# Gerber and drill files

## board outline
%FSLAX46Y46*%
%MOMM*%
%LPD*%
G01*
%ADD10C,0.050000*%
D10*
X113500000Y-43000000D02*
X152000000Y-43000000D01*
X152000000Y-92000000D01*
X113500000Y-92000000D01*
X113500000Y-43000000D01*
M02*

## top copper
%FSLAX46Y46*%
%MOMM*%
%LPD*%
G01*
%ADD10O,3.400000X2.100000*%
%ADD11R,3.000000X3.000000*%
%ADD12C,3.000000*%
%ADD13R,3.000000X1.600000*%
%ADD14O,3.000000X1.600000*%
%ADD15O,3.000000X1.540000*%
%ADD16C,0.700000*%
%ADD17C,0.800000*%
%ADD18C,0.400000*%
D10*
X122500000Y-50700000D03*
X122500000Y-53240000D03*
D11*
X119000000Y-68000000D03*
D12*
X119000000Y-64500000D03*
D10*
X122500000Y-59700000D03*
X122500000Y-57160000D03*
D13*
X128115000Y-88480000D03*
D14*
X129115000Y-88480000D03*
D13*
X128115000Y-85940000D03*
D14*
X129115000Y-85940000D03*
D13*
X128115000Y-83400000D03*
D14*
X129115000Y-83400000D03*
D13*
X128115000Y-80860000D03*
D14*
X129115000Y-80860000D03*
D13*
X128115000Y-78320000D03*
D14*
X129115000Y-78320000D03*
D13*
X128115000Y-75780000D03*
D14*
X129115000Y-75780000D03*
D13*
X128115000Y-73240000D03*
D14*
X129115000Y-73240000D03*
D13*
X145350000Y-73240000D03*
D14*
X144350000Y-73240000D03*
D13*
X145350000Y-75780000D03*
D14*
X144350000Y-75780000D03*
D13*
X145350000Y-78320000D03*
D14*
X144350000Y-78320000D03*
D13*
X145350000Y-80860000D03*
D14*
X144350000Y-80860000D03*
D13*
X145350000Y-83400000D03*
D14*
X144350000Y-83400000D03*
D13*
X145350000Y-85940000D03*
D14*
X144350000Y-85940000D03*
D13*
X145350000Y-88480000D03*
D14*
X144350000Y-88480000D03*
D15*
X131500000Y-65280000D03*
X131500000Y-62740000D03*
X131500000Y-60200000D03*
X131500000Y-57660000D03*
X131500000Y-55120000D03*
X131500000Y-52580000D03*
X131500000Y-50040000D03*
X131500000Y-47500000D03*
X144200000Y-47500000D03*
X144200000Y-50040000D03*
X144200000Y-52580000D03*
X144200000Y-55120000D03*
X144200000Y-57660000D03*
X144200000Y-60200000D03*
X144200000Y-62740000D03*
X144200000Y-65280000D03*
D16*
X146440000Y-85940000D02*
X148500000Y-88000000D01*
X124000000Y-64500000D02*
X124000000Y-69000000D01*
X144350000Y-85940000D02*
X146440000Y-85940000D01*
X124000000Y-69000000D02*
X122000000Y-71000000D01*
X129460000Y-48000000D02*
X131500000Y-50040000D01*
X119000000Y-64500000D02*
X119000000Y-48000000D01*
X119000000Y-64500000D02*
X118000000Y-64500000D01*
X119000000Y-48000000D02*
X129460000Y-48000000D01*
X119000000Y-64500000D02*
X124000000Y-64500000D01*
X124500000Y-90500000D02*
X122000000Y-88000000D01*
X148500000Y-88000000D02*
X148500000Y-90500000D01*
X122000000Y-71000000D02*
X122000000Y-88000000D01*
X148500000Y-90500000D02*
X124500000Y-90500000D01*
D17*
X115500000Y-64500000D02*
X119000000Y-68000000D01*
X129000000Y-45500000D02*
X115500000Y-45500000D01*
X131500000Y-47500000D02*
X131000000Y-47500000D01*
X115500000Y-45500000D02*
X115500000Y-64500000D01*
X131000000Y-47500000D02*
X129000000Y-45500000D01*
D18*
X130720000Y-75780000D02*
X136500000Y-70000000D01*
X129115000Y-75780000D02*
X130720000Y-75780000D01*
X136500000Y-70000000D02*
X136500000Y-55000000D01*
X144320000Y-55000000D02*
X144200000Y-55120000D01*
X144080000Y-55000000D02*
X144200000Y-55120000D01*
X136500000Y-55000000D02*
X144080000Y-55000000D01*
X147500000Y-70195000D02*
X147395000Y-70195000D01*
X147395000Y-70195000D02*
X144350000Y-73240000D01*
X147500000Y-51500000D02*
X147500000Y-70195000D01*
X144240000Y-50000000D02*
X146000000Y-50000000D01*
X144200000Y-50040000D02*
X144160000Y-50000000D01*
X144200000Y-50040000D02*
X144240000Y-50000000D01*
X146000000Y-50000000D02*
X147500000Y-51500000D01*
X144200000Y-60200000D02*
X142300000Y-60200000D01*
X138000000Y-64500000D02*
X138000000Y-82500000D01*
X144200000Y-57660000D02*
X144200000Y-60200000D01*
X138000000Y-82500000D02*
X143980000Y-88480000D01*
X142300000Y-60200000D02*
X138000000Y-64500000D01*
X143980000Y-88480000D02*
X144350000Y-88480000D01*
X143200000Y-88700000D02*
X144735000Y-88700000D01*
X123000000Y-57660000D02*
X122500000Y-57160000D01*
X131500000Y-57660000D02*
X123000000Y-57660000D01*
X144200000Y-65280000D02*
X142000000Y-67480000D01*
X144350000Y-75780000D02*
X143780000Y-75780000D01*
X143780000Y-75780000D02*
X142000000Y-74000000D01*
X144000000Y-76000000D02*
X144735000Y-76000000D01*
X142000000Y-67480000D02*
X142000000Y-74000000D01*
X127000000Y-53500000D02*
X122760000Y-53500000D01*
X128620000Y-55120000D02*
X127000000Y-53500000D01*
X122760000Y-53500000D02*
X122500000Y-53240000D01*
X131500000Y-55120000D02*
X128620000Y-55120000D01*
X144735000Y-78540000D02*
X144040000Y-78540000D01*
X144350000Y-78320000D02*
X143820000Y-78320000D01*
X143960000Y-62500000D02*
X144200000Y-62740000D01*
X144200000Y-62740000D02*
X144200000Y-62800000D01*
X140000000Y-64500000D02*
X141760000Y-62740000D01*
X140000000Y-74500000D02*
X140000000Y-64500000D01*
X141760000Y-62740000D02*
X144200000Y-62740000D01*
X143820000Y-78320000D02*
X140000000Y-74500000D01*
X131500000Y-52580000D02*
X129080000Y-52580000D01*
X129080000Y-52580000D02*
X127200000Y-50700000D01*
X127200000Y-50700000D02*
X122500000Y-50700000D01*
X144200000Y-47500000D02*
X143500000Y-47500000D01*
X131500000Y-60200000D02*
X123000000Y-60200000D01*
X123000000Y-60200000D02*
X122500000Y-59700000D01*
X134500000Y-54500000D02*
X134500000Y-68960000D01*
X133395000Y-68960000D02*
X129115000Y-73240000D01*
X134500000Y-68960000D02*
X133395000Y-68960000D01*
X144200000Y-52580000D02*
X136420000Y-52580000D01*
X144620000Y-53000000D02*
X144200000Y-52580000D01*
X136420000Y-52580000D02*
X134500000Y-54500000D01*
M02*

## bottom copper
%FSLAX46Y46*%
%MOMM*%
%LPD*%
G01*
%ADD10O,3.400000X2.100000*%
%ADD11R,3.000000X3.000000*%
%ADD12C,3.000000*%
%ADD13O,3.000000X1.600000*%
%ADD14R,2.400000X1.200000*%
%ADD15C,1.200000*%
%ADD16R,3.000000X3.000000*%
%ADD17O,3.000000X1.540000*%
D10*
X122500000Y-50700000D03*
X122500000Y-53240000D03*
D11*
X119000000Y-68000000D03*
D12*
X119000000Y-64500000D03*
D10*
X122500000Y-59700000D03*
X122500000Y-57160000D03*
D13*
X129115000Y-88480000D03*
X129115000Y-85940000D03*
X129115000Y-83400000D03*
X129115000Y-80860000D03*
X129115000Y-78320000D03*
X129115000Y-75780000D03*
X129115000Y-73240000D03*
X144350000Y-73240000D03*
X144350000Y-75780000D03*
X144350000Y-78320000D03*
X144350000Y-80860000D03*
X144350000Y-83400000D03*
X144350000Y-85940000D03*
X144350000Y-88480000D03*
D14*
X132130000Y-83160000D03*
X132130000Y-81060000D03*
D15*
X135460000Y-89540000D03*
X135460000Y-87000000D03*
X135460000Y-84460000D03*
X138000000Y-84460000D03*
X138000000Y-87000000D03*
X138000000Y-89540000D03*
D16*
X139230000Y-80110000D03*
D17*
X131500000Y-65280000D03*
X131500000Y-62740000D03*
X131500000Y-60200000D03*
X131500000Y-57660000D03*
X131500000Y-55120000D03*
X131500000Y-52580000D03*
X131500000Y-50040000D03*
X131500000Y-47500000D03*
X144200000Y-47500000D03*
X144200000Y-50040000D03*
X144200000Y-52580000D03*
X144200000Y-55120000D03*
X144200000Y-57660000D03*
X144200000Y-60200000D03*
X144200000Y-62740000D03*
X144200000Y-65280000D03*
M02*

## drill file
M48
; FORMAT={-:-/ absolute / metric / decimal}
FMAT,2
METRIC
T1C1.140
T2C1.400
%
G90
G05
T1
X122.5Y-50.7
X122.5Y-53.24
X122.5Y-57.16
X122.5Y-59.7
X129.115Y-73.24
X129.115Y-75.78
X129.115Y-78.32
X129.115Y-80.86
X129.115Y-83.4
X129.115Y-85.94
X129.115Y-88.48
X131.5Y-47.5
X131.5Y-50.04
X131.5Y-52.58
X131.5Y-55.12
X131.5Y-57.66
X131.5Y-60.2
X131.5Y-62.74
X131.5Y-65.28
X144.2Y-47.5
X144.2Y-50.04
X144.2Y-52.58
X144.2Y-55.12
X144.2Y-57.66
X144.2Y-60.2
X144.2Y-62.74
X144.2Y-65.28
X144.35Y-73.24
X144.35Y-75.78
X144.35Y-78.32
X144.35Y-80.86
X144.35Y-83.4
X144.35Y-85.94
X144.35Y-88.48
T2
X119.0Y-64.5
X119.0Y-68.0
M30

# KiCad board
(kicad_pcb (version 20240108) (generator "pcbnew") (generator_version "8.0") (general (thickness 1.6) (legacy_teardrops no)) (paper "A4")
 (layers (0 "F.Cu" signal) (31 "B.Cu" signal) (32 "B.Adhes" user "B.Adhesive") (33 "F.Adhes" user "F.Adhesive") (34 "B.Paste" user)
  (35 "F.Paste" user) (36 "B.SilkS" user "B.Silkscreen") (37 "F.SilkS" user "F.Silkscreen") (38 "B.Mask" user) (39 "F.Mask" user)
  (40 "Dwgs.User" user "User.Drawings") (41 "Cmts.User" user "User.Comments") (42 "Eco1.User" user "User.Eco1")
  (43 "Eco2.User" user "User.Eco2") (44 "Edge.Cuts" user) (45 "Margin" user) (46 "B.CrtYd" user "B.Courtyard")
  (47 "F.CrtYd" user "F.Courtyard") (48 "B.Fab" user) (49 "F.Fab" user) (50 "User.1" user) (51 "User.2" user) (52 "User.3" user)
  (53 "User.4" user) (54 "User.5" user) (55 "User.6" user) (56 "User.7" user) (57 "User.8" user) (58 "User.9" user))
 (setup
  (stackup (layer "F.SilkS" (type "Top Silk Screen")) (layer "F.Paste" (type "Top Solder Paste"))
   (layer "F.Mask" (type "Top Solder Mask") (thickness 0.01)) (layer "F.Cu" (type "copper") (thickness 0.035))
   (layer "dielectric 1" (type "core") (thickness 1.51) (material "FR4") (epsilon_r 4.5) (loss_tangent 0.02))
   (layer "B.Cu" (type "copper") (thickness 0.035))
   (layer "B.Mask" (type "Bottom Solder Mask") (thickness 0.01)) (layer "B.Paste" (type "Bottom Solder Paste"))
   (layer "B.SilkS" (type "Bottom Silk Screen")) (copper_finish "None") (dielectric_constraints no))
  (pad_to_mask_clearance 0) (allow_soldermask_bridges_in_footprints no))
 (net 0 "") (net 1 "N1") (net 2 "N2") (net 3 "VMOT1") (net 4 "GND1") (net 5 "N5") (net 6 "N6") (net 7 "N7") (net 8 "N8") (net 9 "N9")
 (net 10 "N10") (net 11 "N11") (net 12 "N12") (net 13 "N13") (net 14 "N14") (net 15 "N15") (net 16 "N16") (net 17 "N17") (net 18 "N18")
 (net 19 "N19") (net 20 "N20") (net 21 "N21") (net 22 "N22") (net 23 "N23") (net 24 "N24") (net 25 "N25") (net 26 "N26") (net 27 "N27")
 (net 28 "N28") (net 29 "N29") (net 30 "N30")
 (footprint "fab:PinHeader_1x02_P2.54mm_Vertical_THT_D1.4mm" (layer "F.Cu") (at 122.5 50.7)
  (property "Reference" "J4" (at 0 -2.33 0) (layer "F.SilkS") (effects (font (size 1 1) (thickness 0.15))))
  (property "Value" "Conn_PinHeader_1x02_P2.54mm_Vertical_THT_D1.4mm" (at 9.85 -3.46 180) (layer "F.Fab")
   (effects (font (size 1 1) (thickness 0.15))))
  (pad "1" thru_hole oval (at 0 0) (size 3.4 2.1) (drill 1.14) (layers "*.Cu" "*.Mask") (remove_unused_layers no) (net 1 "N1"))
  (pad "2" thru_hole oval (at 0 2.54) (size 3.4 2.1) (drill 1.14) (layers "*.Cu" "*.Mask") (remove_unused_layers no) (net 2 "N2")))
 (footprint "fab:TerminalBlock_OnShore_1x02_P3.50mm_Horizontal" (layer "F.Cu") (at 119 68 90)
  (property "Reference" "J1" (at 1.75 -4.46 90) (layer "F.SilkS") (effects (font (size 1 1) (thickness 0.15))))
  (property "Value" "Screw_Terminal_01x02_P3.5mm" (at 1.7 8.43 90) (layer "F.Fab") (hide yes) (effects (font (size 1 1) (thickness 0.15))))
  (pad "1" thru_hole rect (at 0 0 90) (size 3 3) (drill 1.4) (layers "*.Cu" "*.Mask") (remove_unused_layers no) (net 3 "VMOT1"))
  (pad "2" thru_hole circle (at 3.5 0 90) (size 3 3) (drill 1.4) (layers "*.Cu" "*.Mask") (remove_unused_layers no) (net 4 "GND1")))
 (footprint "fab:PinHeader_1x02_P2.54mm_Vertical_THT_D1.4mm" (layer "F.Cu") (at 122.5 59.7 180)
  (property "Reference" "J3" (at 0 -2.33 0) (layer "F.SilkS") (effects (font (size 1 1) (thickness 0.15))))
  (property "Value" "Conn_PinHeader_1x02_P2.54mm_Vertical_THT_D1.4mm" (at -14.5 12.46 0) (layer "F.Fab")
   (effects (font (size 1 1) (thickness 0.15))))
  (pad "1" thru_hole oval (at 0 0 180) (size 3.4 2.1) (drill 1.14) (layers "*.Cu" "*.Mask") (remove_unused_layers no) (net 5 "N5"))
  (pad "2" thru_hole oval (at 0 2.54 180) (size 3.4 2.1) (drill 1.14) (layers "*.Cu" "*.Mask") (remove_unused_layers no) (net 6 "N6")))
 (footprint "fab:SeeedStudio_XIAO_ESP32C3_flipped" (layer "B.Cu") (at 136.73 80.86)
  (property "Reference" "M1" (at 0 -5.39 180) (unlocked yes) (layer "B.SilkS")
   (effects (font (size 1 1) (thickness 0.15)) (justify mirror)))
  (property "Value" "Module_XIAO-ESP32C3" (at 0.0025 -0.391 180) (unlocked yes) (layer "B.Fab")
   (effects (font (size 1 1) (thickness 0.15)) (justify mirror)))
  (pad "1" smd rect (at -7.615 7.62) (size 3 1.6) (drill (offset -1 0)) (layers "F.Cu" "F.Paste" "F.Mask") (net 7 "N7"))
  (pad "1" thru_hole oval (at -7.615 7.62) (size 3 1.6) (drill 1.14) (layers "*.Cu" "*.Mask") (remove_unused_layers no) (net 7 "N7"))
  (pad "2" smd rect (at -7.615 5.08) (size 3 1.6) (drill (offset -1 0)) (layers "F.Cu" "F.Paste" "F.Mask") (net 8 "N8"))
  (pad "2" thru_hole oval (at -7.615 5.08) (size 3 1.6) (drill 1.14) (layers "*.Cu" "*.Mask") (remove_unused_layers no) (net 8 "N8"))
  (pad "3" smd rect (at -7.615 2.54) (size 3 1.6) (drill (offset -1 0)) (layers "F.Cu" "F.Paste" "F.Mask") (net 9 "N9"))
  (pad "3" thru_hole oval (at -7.615 2.54) (size 3 1.6) (drill 1.14) (layers "*.Cu" "*.Mask") (remove_unused_layers no) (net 9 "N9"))
  (pad "4" smd rect (at -7.615 0) (size 3 1.6) (drill (offset -1 0)) (layers "F.Cu" "F.Paste" "F.Mask") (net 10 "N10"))
  (pad "4" thru_hole oval (at -7.615 0) (size 3 1.6) (drill 1.14) (layers "*.Cu" "*.Mask") (remove_unused_layers no) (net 10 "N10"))
  (pad "5" smd rect (at -7.615 -2.54) (size 3 1.6) (drill (offset -1 0)) (layers "F.Cu" "F.Paste" "F.Mask") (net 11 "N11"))
  (pad "5" thru_hole oval (at -7.615 -2.54) (size 3 1.6) (drill 1.14) (layers "*.Cu" "*.Mask") (remove_unused_layers no) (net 11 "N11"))
  (pad "6" smd rect (at -7.615 -5.08) (size 3 1.6) (drill (offset -1 0)) (layers "F.Cu" "F.Paste" "F.Mask") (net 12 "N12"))
  (pad "6" thru_hole oval (at -7.615 -5.08) (size 3 1.6) (drill 1.14) (layers "*.Cu" "*.Mask") (remove_unused_layers no) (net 12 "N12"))
  (pad "7" smd rect (at -7.615 -7.62) (size 3 1.6) (drill (offset -1 0)) (layers "F.Cu" "F.Paste" "F.Mask") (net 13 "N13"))
  (pad "7" thru_hole oval (at -7.615 -7.62) (size 3 1.6) (drill 1.14) (layers "*.Cu" "*.Mask") (remove_unused_layers no) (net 13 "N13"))
  (pad "8" smd rect (at 7.62 -7.62) (size 3 1.6) (drill (offset 1 0)) (layers "F.Cu" "F.Paste" "F.Mask") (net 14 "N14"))
  (pad "8" thru_hole oval (at 7.62 -7.62) (size 3 1.6) (drill 1.14) (layers "*.Cu" "*.Mask") (remove_unused_layers no) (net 14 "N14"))
  (pad "9" smd rect (at 7.62 -5.08) (size 3 1.6) (drill (offset 1 0)) (layers "F.Cu" "F.Paste" "F.Mask") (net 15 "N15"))
  (pad "9" thru_hole oval (at 7.62 -5.08) (size 3 1.6) (drill 1.14) (layers "*.Cu" "*.Mask") (remove_unused_layers no) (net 15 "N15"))
  (pad "10" smd rect (at 7.62 -2.54) (size 3 1.6) (drill (offset 1 0)) (layers "F.Cu" "F.Paste" "F.Mask") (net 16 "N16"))
  (pad "10" thru_hole oval (at 7.62 -2.54) (size 3 1.6) (drill 1.14) (layers "*.Cu" "*.Mask") (remove_unused_layers no) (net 16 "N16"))
  (pad "11" smd rect (at 7.62 0) (size 3 1.6) (drill (offset 1 0)) (layers "F.Cu" "F.Paste" "F.Mask") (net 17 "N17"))
  (pad "11" thru_hole oval (at 7.62 0) (size 3 1.6) (drill 1.14) (layers "*.Cu" "*.Mask") (remove_unused_layers no) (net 17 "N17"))
  (pad "12" smd rect (at 7.62 2.54) (size 3 1.6) (drill (offset 1 0)) (layers "F.Cu" "F.Paste" "F.Mask") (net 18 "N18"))
  (pad "12" thru_hole oval (at 7.62 2.54) (size 3 1.6) (drill 1.14) (layers "*.Cu" "*.Mask") (remove_unused_layers no) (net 18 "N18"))
  (pad "13" smd rect (at 7.62 5.08) (size 3 1.6) (drill (offset 1 0)) (layers "F.Cu" "F.Paste" "F.Mask") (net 4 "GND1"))
  (pad "13" thru_hole oval (at 7.62 5.08) (size 3 1.6) (drill 1.14) (layers "*.Cu" "*.Mask") (remove_unused_layers no) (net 4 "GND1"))
  (pad "14" smd rect (at 7.62 7.62) (size 3 1.6) (drill (offset 1 0)) (layers "F.Cu" "F.Paste" "F.Mask") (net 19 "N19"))
  (pad "14" thru_hole oval (at 7.62 7.62) (size 3 1.6) (drill 1.14) (layers "*.Cu" "*.Mask") (remove_unused_layers no) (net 19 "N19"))
  (pad "15" smd rect (at -4.6 2.3) (size 2.4 1.2) (layers "B.Cu" "B.Paste" "B.Mask") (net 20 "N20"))
  (pad "16" smd rect (at -4.6 0.2) (size 2.4 1.2) (layers "B.Cu" "B.Paste" "B.Mask") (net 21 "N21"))
  (pad "17" smd circle (at -1.27 8.68) (size 1.2 1.2) (layers "B.Cu" "B.Paste" "B.Mask") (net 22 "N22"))
  (pad "18" smd circle (at -1.27 6.14) (size 1.2 1.2) (layers "B.Cu" "B.Paste" "B.Mask") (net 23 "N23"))
  (pad "19" smd circle (at -1.27 3.6) (size 1.2 1.2) (layers "B.Cu" "B.Paste" "B.Mask") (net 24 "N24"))
  (pad "20" smd circle (at 1.27 3.6) (size 1.2 1.2) (layers "B.Cu" "B.Paste" "B.Mask") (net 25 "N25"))
  (pad "21" smd circle (at 1.27 6.14) (size 1.2 1.2) (layers "B.Cu" "B.Paste" "B.Mask") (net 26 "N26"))
  (pad "22" smd circle (at 1.27 8.68) (size 1.2 1.2) (layers "B.Cu" "B.Paste" "B.Mask") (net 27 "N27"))
  (pad "23" smd rect (at 2.5 -0.75) (size 3 3) (layers "B.Cu" "B.Paste" "B.Mask") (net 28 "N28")))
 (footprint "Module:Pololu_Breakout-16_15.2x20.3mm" (layer "B.Cu") (at 131.5 65.28)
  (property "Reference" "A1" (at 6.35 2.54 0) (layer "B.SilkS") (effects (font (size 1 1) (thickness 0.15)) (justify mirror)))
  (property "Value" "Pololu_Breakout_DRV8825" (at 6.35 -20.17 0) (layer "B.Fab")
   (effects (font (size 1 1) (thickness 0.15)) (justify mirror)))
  (pad "1" thru_hole oval (at 0 0) (size 3 1.54) (drill 1.14) (layers "*.Cu" "*.Mask") (remove_unused_layers no) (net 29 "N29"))
  (pad "2" thru_hole oval (at 0 -2.54) (size 3 1.54) (drill 1.14) (layers "*.Cu" "*.Mask") (remove_unused_layers no) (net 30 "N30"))
  (pad "3" thru_hole oval (at 0 -5.08) (size 3 1.54) (drill 1.14) (layers "*.Cu" "*.Mask") (remove_unused_layers no) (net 5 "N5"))
  (pad "4" thru_hole oval (at 0 -7.62) (size 3 1.54) (drill 1.14) (layers "*.Cu" "*.Mask") (remove_unused_layers no) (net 6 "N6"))
  (pad "5" thru_hole oval (at 0 -10.16) (size 3 1.54) (drill 1.14) (layers "*.Cu" "*.Mask") (remove_unused_layers no) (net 2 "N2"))
  (pad "6" thru_hole oval (at 0 -12.7) (size 3 1.54) (drill 1.14) (layers "*.Cu" "*.Mask") (remove_unused_layers no) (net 1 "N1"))
  (pad "7" thru_hole oval (at 0 -15.24) (size 3 1.54) (drill 1.14) (layers "*.Cu" "*.Mask") (remove_unused_layers no) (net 4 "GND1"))
  (pad "8" thru_hole oval (at 0 -17.78) (size 3 1.54) (drill 1.14) (layers "*.Cu" "*.Mask") (remove_unused_layers no) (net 3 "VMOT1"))
  (pad "9" thru_hole oval (at 12.7 -17.78) (size 3 1.54) (drill 1.14) (layers "*.Cu" "*.Mask") (remove_unused_layers no) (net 17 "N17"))
  (pad "10" thru_hole oval (at 12.7 -15.24) (size 3 1.54) (drill 1.14) (layers "*.Cu" "*.Mask") (remove_unused_layers no) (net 14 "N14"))
  (pad "11" thru_hole oval (at 12.7 -12.7) (size 3 1.54) (drill 1.14) (layers "*.Cu" "*.Mask") (remove_unused_layers no) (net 13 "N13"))
  (pad "12" thru_hole oval (at 12.7 -10.16) (size 3 1.54) (drill 1.14) (layers "*.Cu" "*.Mask") (remove_unused_layers no) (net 12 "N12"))
  (pad "13" thru_hole oval (at 12.7 -7.62) (size 3 1.54) (drill 1.14) (layers "*.Cu" "*.Mask") (remove_unused_layers no) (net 19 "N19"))
  (pad "14" thru_hole oval (at 12.7 -5.08) (size 3 1.54) (drill 1.14) (layers "*.Cu" "*.Mask") (remove_unused_layers no) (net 19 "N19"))
  (pad "15" thru_hole oval (at 12.7 -2.54) (size 3 1.54) (drill 1.14) (layers "*.Cu" "*.Mask") (remove_unused_layers no) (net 16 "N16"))
  (pad "16" thru_hole oval (at 12.7 0) (size 3 1.54) (drill 1.14) (layers "*.Cu" "*.Mask") (remove_unused_layers no) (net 15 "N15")))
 (gr_rect (start 113.5 43) (end 152 92) (stroke (width 0.05) (type default)) (fill none) (layer "Edge.Cuts"))
 (segment (start 146.44 85.94) (end 148.5 88) (width 0.7) (layer "F.Cu") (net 4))
 (segment (start 124 64.5) (end 124 69) (width 0.7) (layer "F.Cu") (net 4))
 (segment (start 144.35 85.94) (end 146.44 85.94) (width 0.7) (layer "F.Cu") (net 4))
 (segment (start 124 69) (end 122 71) (width 0.7) (layer "F.Cu") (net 4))
 (segment (start 129.46 48) (end 131.5 50.04) (width 0.7) (layer "F.Cu") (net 4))
 (segment (start 119 64.5) (end 119 48) (width 0.7) (layer "F.Cu") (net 4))
 (segment (start 119 64.5) (end 118 64.5) (width 0.7) (layer "F.Cu") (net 4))
 (segment (start 119 48) (end 129.46 48) (width 0.7) (layer "F.Cu") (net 4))
 (segment (start 119 64.5) (end 124 64.5) (width 0.7) (layer "F.Cu") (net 4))
 (segment (start 124.5 90.5) (end 122 88) (width 0.7) (layer "F.Cu") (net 4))
 (segment (start 148.5 88) (end 148.5 90.5) (width 0.7) (layer "F.Cu") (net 4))
 (segment (start 122 71) (end 122 88) (width 0.7) (layer "F.Cu") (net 4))
 (segment (start 148.5 90.5) (end 124.5 90.5) (width 0.7) (layer "F.Cu") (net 4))
 (segment (start 115.5 64.5) (end 119 68) (width 0.8) (layer "F.Cu") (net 3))
 (segment (start 129 45.5) (end 115.5 45.5) (width 0.8) (layer "F.Cu") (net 3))
 (segment (start 131.5 47.5) (end 131 47.5) (width 0.8) (layer "F.Cu") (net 3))
 (segment (start 115.5 45.5) (end 115.5 64.5) (width 0.8) (layer "F.Cu") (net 3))
 (segment (start 131 47.5) (end 129 45.5) (width 0.8) (layer "F.Cu") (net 3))
 (segment (start 130.72 75.78) (end 136.5 70) (width 0.4) (layer "F.Cu") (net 12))
 (segment (start 129.115 75.78) (end 130.72 75.78) (width 0.4) (layer "F.Cu") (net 12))
 (segment (start 136.5 70) (end 136.5 55) (width 0.4) (layer "F.Cu") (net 12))
 (segment (start 144.32 55) (end 144.2 55.12) (width 0.4) (layer "F.Cu") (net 12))
 (segment (start 144.08 55) (end 144.2 55.12) (width 0.4) (layer "F.Cu") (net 12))
 (segment (start 136.5 55) (end 144.08 55) (width 0.4) (layer "F.Cu") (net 12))
 (segment (start 147.5 70.195) (end 147.395 70.195) (width 0.4) (layer "F.Cu") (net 14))
 (segment (start 147.395 70.195) (end 144.35 73.24) (width 0.4) (layer "F.Cu") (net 14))
 (segment (start 147.5 51.5) (end 147.5 70.195) (width 0.4) (layer "F.Cu") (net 14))
 (segment (start 144.24 50) (end 146 50) (width 0.4) (layer "F.Cu") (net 14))
 (segment (start 144.2 50.04) (end 144.16 50) (width 0.4) (layer "F.Cu") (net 14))
 (segment (start 144.2 50.04) (end 144.24 50) (width 0.4) (layer "F.Cu") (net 14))
 (segment (start 146 50) (end 147.5 51.5) (width 0.4) (layer "F.Cu") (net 14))
 (segment (start 144.2 60.2) (end 142.3 60.2) (width 0.4) (layer "F.Cu") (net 19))
 (segment (start 138 64.5) (end 138 82.5) (width 0.4) (layer "F.Cu") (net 19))
 (segment (start 144.2 57.66) (end 144.2 60.2) (width 0.4) (layer "F.Cu") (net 19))
 (segment (start 138 82.5) (end 143.98 88.48) (width 0.4) (layer "F.Cu") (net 19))
 (segment (start 142.3 60.2) (end 138 64.5) (width 0.4) (layer "F.Cu") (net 19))
 (segment (start 143.98 88.48) (end 144.35 88.48) (width 0.4) (layer "F.Cu") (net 19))
 (segment (start 143.2 88.7) (end 144.735 88.7) (width 0.4) (layer "F.Cu") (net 19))
 (segment (start 123 57.66) (end 122.5 57.16) (width 0.4) (layer "F.Cu") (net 6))
 (segment (start 131.5 57.66) (end 123 57.66) (width 0.4) (layer "F.Cu") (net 6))
 (segment (start 144.2 65.28) (end 142 67.48) (width 0.4) (layer "F.Cu") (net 15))
 (segment (start 144.35 75.78) (end 143.78 75.78) (width 0.4) (layer "F.Cu") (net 15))
 (segment (start 143.78 75.78) (end 142 74) (width 0.4) (layer "F.Cu") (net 15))
 (segment (start 144 76) (end 144.735 76) (width 0.4) (layer "F.Cu") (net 15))
 (segment (start 142 67.48) (end 142 74) (width 0.4) (layer "F.Cu") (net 15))
 (segment (start 127 53.5) (end 122.76 53.5) (width 0.4) (layer "F.Cu") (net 2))
 (segment (start 128.62 55.12) (end 127 53.5) (width 0.4) (layer "F.Cu") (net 2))
 (segment (start 122.76 53.5) (end 122.5 53.24) (width 0.4) (layer "F.Cu") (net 2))
 (segment (start 131.5 55.12) (end 128.62 55.12) (width 0.4) (layer "F.Cu") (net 2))
 (segment (start 144.735 78.54) (end 144.04 78.54) (width 0.4) (layer "F.Cu") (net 16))
 (segment (start 144.35 78.32) (end 143.82 78.32) (width 0.4) (layer "F.Cu") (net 16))
 (segment (start 143.96 62.5) (end 144.2 62.74) (width 0.4) (layer "F.Cu") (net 16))
 (segment (start 144.2 62.74) (end 144.2 62.8) (width 0.4) (layer "F.Cu") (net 16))
 (segment (start 140 64.5) (end 141.76 62.74) (width 0.4) (layer "F.Cu") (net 16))
 (segment (start 140 74.5) (end 140 64.5) (width 0.4) (layer "F.Cu") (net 16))
 (segment (start 141.76 62.74) (end 144.2 62.74) (width 0.4) (layer "F.Cu") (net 16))
 (segment (start 143.82 78.32) (end 140 74.5) (width 0.4) (layer "F.Cu") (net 16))
 (segment (start 131.5 52.58) (end 129.08 52.58) (width 0.4) (layer "F.Cu") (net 1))
 (segment (start 129.08 52.58) (end 127.2 50.7) (width 0.4) (layer "F.Cu") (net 1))
 (segment (start 127.2 50.7) (end 122.5 50.7) (width 0.4) (layer "F.Cu") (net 1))
 (segment (start 144.2 47.5) (end 143.5 47.5) (width 0.4) (layer "F.Cu") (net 17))
 (segment (start 131.5 60.2) (end 123 60.2) (width 0.4) (layer "F.Cu") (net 5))
 (segment (start 123 60.2) (end 122.5 59.7) (width 0.4) (layer "F.Cu") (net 5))
 (segment (start 134.5 54.5) (end 134.5 68.96) (width 0.4) (layer "F.Cu") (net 13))
 (segment (start 133.395 68.96) (end 129.115 73.24) (width 0.4) (layer "F.Cu") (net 13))
 (segment (start 134.5 68.96) (end 133.395 68.96) (width 0.4) (layer "F.Cu") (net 13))
 (segment (start 144.2 52.58) (end 136.42 52.58) (width 0.4) (layer "F.Cu") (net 13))
 (segment (start 144.62 53) (end 144.2 52.58) (width 0.4) (layer "F.Cu") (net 13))
 (segment (start 136.42 52.58) (end 134.5 54.5) (width 0.4) (layer "F.Cu") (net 13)))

